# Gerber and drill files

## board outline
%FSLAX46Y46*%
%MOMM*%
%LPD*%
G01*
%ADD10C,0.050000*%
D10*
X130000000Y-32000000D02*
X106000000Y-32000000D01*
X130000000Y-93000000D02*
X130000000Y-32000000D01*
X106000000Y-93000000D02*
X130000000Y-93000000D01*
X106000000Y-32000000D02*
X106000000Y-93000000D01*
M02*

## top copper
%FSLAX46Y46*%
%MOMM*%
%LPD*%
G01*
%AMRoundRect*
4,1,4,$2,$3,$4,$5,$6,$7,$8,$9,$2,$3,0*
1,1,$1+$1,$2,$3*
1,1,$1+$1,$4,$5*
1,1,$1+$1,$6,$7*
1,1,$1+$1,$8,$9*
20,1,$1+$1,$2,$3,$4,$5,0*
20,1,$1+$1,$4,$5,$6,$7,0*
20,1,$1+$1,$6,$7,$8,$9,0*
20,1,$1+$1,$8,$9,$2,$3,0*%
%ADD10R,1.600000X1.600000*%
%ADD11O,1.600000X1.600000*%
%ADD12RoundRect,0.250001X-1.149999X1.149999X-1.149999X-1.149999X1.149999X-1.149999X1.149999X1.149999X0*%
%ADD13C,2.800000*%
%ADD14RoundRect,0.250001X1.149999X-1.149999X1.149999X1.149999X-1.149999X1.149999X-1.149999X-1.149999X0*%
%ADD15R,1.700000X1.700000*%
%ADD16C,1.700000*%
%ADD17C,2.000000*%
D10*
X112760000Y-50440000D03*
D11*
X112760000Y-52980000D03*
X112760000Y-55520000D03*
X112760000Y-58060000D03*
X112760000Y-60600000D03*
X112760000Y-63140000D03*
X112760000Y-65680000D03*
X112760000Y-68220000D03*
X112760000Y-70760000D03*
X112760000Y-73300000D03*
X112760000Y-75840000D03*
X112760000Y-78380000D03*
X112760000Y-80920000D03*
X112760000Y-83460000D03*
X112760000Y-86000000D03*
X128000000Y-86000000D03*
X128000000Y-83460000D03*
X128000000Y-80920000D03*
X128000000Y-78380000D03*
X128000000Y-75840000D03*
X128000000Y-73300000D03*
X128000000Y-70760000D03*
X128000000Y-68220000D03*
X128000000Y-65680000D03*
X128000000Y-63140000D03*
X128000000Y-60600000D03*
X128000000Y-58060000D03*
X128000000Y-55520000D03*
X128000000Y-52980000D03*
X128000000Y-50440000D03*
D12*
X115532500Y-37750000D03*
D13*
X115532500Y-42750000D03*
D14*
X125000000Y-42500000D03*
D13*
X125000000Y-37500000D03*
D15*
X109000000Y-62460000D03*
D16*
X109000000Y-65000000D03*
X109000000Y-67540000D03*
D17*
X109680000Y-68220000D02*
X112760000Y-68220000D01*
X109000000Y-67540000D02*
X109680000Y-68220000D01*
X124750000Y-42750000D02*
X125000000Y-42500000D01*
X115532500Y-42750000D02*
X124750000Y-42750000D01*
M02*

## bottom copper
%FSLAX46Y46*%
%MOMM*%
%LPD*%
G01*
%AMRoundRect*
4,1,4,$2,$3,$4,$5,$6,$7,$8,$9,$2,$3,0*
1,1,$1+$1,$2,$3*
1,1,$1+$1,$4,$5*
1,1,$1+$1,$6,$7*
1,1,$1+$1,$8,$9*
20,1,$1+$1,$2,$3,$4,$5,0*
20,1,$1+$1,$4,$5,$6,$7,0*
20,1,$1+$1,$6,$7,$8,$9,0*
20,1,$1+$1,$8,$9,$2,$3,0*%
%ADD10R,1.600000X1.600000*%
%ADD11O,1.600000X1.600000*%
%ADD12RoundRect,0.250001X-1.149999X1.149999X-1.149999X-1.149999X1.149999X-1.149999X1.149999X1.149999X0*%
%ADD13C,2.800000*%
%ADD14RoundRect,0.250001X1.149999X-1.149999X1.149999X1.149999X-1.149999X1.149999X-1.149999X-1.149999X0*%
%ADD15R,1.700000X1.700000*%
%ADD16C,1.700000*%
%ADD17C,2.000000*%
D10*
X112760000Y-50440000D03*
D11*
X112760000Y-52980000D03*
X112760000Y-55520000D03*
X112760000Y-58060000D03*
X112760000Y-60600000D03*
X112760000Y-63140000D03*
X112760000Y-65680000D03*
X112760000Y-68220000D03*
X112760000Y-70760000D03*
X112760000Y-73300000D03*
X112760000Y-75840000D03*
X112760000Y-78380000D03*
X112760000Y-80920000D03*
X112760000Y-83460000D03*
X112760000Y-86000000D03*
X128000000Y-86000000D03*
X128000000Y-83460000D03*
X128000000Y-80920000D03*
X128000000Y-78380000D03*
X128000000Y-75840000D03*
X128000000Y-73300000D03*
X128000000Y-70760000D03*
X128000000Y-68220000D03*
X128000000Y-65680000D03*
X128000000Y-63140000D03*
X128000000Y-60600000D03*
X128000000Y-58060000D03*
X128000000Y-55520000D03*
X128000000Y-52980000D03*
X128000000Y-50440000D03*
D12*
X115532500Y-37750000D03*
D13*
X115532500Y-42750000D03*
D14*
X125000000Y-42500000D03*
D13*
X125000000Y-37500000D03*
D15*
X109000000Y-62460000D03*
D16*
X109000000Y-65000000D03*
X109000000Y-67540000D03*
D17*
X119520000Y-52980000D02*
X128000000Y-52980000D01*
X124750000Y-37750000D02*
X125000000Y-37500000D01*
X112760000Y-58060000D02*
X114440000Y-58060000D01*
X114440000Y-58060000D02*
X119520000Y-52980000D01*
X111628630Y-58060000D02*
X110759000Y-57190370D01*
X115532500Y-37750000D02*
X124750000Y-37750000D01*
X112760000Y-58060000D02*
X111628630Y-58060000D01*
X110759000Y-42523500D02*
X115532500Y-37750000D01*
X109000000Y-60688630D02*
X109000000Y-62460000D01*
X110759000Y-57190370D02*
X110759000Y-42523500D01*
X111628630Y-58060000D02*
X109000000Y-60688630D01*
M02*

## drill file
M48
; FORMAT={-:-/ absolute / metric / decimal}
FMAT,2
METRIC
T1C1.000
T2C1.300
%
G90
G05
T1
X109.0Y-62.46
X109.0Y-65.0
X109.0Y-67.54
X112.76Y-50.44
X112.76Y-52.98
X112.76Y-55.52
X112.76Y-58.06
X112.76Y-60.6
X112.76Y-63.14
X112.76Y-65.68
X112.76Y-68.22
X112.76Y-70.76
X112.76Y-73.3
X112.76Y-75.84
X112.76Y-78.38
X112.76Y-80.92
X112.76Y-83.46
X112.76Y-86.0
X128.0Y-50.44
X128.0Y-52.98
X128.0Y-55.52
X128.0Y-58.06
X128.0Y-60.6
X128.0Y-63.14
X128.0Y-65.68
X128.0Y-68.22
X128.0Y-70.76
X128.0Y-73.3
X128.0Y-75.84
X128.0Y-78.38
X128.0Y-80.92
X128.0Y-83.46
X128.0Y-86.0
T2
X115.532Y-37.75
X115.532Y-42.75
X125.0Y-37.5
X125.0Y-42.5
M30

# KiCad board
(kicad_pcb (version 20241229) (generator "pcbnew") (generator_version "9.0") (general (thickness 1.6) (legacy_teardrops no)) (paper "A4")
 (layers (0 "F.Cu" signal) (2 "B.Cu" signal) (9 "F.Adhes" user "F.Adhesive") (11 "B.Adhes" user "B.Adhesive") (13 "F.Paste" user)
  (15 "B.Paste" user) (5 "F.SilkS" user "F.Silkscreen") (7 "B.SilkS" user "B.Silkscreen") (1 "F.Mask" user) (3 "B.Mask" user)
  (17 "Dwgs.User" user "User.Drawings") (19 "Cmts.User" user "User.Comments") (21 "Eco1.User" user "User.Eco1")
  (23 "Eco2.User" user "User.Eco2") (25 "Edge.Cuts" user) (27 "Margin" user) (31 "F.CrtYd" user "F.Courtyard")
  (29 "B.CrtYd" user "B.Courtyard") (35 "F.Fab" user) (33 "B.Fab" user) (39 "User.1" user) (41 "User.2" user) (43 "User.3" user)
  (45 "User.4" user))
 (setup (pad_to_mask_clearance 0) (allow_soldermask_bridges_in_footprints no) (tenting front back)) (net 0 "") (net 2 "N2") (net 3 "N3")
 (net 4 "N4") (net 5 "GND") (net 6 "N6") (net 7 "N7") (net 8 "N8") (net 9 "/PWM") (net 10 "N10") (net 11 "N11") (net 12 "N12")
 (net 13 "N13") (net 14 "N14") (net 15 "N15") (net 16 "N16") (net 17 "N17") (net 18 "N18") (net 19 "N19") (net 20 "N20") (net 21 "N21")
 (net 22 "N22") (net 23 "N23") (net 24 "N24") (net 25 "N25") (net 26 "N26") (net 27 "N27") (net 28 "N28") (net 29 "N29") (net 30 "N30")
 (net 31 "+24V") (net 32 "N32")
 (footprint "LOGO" (layer "F.Cu") (at 107 88 90)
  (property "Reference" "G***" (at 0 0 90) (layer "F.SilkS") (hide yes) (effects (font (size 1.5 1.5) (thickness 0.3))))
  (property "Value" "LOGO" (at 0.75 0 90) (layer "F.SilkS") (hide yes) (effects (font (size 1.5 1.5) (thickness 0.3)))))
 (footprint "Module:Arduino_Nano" (layer "F.Cu") (at 112.76 50.44)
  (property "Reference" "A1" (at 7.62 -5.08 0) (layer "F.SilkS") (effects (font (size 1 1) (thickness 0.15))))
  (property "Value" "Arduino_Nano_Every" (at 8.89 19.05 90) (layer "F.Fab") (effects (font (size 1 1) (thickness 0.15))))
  (pad "1" thru_hole rect (at 0 0) (size 1.6 1.6) (drill 1) (layers "*.Cu" "*.Mask") (remove_unused_layers no) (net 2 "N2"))
  (pad "2" thru_hole oval (at 0 2.54) (size 1.6 1.6) (drill 1) (layers "*.Cu" "*.Mask") (remove_unused_layers no) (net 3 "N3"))
  (pad "3" thru_hole oval (at 0 5.08) (size 1.6 1.6) (drill 1) (layers "*.Cu" "*.Mask") (remove_unused_layers no) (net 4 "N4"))
  (pad "4" thru_hole oval (at 0 7.62) (size 1.6 1.6) (drill 1) (layers "*.Cu" "*.Mask") (remove_unused_layers no) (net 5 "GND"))
  (pad "5" thru_hole oval (at 0 10.16) (size 1.6 1.6) (drill 1) (layers "*.Cu" "*.Mask") (remove_unused_layers no) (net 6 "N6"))
  (pad "6" thru_hole oval (at 0 12.7) (size 1.6 1.6) (drill 1) (layers "*.Cu" "*.Mask") (remove_unused_layers no) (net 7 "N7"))
  (pad "7" thru_hole oval (at 0 15.24) (size 1.6 1.6) (drill 1) (layers "*.Cu" "*.Mask") (remove_unused_layers no) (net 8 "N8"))
  (pad "8" thru_hole oval (at 0 17.78) (size 1.6 1.6) (drill 1) (layers "*.Cu" "*.Mask") (remove_unused_layers no) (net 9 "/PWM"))
  (pad "9" thru_hole oval (at 0 20.32) (size 1.6 1.6) (drill 1) (layers "*.Cu" "*.Mask") (remove_unused_layers no) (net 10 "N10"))
  (pad "10" thru_hole oval (at 0 22.86) (size 1.6 1.6) (drill 1) (layers "*.Cu" "*.Mask") (remove_unused_layers no) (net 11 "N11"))
  (pad "11" thru_hole oval (at 0 25.4) (size 1.6 1.6) (drill 1) (layers "*.Cu" "*.Mask") (remove_unused_layers no) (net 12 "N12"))
  (pad "12" thru_hole oval (at 0 27.94) (size 1.6 1.6) (drill 1) (layers "*.Cu" "*.Mask") (remove_unused_layers no) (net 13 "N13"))
  (pad "13" thru_hole oval (at 0 30.48) (size 1.6 1.6) (drill 1) (layers "*.Cu" "*.Mask") (remove_unused_layers no) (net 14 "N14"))
  (pad "14" thru_hole oval (at 0 33.02) (size 1.6 1.6) (drill 1) (layers "*.Cu" "*.Mask") (remove_unused_layers no) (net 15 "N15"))
  (pad "15" thru_hole oval (at 0 35.56) (size 1.6 1.6) (drill 1) (layers "*.Cu" "*.Mask") (remove_unused_layers no) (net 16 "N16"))
  (pad "16" thru_hole oval (at 15.24 35.56) (size 1.6 1.6) (drill 1) (layers "*.Cu" "*.Mask") (remove_unused_layers no) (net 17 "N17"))
  (pad "17" thru_hole oval (at 15.24 33.02) (size 1.6 1.6) (drill 1) (layers "*.Cu" "*.Mask") (remove_unused_layers no) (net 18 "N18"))
  (pad "18" thru_hole oval (at 15.24 30.48) (size 1.6 1.6) (drill 1) (layers "*.Cu" "*.Mask") (remove_unused_layers no) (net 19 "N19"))
  (pad "19" thru_hole oval (at 15.24 27.94) (size 1.6 1.6) (drill 1) (layers "*.Cu" "*.Mask") (remove_unused_layers no) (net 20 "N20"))
  (pad "20" thru_hole oval (at 15.24 25.4) (size 1.6 1.6) (drill 1) (layers "*.Cu" "*.Mask") (remove_unused_layers no) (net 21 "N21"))
  (pad "21" thru_hole oval (at 15.24 22.86) (size 1.6 1.6) (drill 1) (layers "*.Cu" "*.Mask") (remove_unused_layers no) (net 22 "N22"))
  (pad "22" thru_hole oval (at 15.24 20.32) (size 1.6 1.6) (drill 1) (layers "*.Cu" "*.Mask") (remove_unused_layers no) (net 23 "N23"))
  (pad "23" thru_hole oval (at 15.24 17.78) (size 1.6 1.6) (drill 1) (layers "*.Cu" "*.Mask") (remove_unused_layers no) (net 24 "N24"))
  (pad "24" thru_hole oval (at 15.24 15.24) (size 1.6 1.6) (drill 1) (layers "*.Cu" "*.Mask") (remove_unused_layers no) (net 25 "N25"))
  (pad "25" thru_hole oval (at 15.24 12.7) (size 1.6 1.6) (drill 1) (layers "*.Cu" "*.Mask") (remove_unused_layers no) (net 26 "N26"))
  (pad "26" thru_hole oval (at 15.24 10.16) (size 1.6 1.6) (drill 1) (layers "*.Cu" "*.Mask") (remove_unused_layers no) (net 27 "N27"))
  (pad "27" thru_hole oval (at 15.24 7.62) (size 1.6 1.6) (drill 1) (layers "*.Cu" "*.Mask") (remove_unused_layers no) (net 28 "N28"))
  (pad "28" thru_hole oval (at 15.24 5.08) (size 1.6 1.6) (drill 1) (layers "*.Cu" "*.Mask") (remove_unused_layers no) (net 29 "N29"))
  (pad "29" thru_hole oval (at 15.24 2.54) (size 1.6 1.6) (drill 1) (layers "*.Cu" "*.Mask") (remove_unused_layers no) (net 5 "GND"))
  (pad "30" thru_hole oval (at 15.24 0) (size 1.6 1.6) (drill 1) (layers "*.Cu" "*.Mask") (remove_unused_layers no) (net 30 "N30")))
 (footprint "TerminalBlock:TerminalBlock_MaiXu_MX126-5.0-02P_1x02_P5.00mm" (layer "F.Cu") (at 115.5325 37.75 -90)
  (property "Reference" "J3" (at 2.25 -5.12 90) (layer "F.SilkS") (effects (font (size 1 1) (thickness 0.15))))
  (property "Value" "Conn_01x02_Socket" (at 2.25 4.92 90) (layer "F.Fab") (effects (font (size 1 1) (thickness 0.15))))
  (pad "1" thru_hole roundrect (at 0 0 270) (size 2.8 2.8) (drill 1.3) (layers "*.Cu" "*.Mask") (remove_unused_layers no)
   (roundrect_rratio 0.089286) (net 5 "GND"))
  (pad "2" thru_hole circle (at 5 0 270) (size 2.8 2.8) (drill 1.3) (layers "*.Cu" "*.Mask") (remove_unused_layers no) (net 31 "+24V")))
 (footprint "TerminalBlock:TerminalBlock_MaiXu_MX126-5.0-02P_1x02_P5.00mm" (layer "F.Cu") (at 125 42.5 90)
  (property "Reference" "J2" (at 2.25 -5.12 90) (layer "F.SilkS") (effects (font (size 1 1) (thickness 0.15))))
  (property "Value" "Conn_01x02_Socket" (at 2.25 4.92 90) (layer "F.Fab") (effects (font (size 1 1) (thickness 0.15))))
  (pad "1" thru_hole roundrect (at 0 0 90) (size 2.8 2.8) (drill 1.3) (layers "*.Cu" "*.Mask") (remove_unused_layers no)
   (roundrect_rratio 0.089286) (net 31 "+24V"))
  (pad "2" thru_hole circle (at 5 0 90) (size 2.8 2.8) (drill 1.3) (layers "*.Cu" "*.Mask") (remove_unused_layers no) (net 5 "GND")))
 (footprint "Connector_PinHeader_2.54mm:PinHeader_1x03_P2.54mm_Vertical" (layer "F.Cu") (at 109 62.46)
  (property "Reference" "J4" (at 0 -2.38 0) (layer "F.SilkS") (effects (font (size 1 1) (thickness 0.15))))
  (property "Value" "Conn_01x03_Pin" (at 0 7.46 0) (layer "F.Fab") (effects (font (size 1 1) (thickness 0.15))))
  (pad "1" thru_hole rect (at 0 0) (size 1.7 1.7) (drill 1) (layers "*.Cu" "*.Mask") (remove_unused_layers no) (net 5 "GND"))
  (pad "2" thru_hole circle (at 0 2.54) (size 1.7 1.7) (drill 1) (layers "*.Cu" "*.Mask") (remove_unused_layers no) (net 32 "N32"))
  (pad "3" thru_hole circle (at 0 5.08) (size 1.7 1.7) (drill 1) (layers "*.Cu" "*.Mask") (remove_unused_layers no) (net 9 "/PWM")))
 (gr_line (start 130 32) (end 106 32) (stroke (width 0.05) (type default)) (layer "Edge.Cuts"))
 (gr_line (start 130 93) (end 130 32) (stroke (width 0.05) (type default)) (layer "Edge.Cuts"))
 (gr_line (start 106 93) (end 130 93) (stroke (width 0.05) (type default)) (layer "Edge.Cuts"))
 (gr_line (start 106 32) (end 106 93) (stroke (width 0.05) (type default)) (layer "Edge.Cuts"))
 (segment (start 109.68 68.22) (end 112.76 68.22) (width 2) (layer "F.Cu") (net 9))
 (segment (start 109 67.54) (end 109.68 68.22) (width 2) (layer "F.Cu") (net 9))
 (segment (start 119.52 52.98) (end 128 52.98) (width 2) (layer "B.Cu") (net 5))
 (segment (start 124.75 37.75) (end 125 37.5) (width 2) (layer "B.Cu") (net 5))
 (segment (start 112.76 58.06) (end 114.44 58.06) (width 2) (layer "B.Cu") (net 5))
 (segment (start 114.44 58.06) (end 119.52 52.98) (width 2) (layer "B.Cu") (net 5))
 (segment (start 111.62863 58.06) (end 110.759 57.19037) (width 2) (layer "B.Cu") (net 5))
 (segment (start 115.5325 37.75) (end 124.75 37.75) (width 2) (layer "B.Cu") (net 5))
 (segment (start 112.76 58.06) (end 111.62863 58.06) (width 2) (layer "B.Cu") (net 5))
 (segment (start 110.759 42.5235) (end 115.5325 37.75) (width 2) (layer "B.Cu") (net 5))
 (segment (start 109 60.68863) (end 109 62.46) (width 2) (layer "B.Cu") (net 5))
 (segment (start 110.759 57.19037) (end 110.759 42.5235) (width 2) (layer "B.Cu") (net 5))
 (segment (start 111.62863 58.06) (end 109 60.68863) (width 2) (layer "B.Cu") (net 5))
 (segment (start 124.75 42.75) (end 125 42.5) (width 2) (layer "F.Cu") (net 31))
 (segment (start 115.5325 42.75) (end 124.75 42.75) (width 2) (layer "F.Cu") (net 31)))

